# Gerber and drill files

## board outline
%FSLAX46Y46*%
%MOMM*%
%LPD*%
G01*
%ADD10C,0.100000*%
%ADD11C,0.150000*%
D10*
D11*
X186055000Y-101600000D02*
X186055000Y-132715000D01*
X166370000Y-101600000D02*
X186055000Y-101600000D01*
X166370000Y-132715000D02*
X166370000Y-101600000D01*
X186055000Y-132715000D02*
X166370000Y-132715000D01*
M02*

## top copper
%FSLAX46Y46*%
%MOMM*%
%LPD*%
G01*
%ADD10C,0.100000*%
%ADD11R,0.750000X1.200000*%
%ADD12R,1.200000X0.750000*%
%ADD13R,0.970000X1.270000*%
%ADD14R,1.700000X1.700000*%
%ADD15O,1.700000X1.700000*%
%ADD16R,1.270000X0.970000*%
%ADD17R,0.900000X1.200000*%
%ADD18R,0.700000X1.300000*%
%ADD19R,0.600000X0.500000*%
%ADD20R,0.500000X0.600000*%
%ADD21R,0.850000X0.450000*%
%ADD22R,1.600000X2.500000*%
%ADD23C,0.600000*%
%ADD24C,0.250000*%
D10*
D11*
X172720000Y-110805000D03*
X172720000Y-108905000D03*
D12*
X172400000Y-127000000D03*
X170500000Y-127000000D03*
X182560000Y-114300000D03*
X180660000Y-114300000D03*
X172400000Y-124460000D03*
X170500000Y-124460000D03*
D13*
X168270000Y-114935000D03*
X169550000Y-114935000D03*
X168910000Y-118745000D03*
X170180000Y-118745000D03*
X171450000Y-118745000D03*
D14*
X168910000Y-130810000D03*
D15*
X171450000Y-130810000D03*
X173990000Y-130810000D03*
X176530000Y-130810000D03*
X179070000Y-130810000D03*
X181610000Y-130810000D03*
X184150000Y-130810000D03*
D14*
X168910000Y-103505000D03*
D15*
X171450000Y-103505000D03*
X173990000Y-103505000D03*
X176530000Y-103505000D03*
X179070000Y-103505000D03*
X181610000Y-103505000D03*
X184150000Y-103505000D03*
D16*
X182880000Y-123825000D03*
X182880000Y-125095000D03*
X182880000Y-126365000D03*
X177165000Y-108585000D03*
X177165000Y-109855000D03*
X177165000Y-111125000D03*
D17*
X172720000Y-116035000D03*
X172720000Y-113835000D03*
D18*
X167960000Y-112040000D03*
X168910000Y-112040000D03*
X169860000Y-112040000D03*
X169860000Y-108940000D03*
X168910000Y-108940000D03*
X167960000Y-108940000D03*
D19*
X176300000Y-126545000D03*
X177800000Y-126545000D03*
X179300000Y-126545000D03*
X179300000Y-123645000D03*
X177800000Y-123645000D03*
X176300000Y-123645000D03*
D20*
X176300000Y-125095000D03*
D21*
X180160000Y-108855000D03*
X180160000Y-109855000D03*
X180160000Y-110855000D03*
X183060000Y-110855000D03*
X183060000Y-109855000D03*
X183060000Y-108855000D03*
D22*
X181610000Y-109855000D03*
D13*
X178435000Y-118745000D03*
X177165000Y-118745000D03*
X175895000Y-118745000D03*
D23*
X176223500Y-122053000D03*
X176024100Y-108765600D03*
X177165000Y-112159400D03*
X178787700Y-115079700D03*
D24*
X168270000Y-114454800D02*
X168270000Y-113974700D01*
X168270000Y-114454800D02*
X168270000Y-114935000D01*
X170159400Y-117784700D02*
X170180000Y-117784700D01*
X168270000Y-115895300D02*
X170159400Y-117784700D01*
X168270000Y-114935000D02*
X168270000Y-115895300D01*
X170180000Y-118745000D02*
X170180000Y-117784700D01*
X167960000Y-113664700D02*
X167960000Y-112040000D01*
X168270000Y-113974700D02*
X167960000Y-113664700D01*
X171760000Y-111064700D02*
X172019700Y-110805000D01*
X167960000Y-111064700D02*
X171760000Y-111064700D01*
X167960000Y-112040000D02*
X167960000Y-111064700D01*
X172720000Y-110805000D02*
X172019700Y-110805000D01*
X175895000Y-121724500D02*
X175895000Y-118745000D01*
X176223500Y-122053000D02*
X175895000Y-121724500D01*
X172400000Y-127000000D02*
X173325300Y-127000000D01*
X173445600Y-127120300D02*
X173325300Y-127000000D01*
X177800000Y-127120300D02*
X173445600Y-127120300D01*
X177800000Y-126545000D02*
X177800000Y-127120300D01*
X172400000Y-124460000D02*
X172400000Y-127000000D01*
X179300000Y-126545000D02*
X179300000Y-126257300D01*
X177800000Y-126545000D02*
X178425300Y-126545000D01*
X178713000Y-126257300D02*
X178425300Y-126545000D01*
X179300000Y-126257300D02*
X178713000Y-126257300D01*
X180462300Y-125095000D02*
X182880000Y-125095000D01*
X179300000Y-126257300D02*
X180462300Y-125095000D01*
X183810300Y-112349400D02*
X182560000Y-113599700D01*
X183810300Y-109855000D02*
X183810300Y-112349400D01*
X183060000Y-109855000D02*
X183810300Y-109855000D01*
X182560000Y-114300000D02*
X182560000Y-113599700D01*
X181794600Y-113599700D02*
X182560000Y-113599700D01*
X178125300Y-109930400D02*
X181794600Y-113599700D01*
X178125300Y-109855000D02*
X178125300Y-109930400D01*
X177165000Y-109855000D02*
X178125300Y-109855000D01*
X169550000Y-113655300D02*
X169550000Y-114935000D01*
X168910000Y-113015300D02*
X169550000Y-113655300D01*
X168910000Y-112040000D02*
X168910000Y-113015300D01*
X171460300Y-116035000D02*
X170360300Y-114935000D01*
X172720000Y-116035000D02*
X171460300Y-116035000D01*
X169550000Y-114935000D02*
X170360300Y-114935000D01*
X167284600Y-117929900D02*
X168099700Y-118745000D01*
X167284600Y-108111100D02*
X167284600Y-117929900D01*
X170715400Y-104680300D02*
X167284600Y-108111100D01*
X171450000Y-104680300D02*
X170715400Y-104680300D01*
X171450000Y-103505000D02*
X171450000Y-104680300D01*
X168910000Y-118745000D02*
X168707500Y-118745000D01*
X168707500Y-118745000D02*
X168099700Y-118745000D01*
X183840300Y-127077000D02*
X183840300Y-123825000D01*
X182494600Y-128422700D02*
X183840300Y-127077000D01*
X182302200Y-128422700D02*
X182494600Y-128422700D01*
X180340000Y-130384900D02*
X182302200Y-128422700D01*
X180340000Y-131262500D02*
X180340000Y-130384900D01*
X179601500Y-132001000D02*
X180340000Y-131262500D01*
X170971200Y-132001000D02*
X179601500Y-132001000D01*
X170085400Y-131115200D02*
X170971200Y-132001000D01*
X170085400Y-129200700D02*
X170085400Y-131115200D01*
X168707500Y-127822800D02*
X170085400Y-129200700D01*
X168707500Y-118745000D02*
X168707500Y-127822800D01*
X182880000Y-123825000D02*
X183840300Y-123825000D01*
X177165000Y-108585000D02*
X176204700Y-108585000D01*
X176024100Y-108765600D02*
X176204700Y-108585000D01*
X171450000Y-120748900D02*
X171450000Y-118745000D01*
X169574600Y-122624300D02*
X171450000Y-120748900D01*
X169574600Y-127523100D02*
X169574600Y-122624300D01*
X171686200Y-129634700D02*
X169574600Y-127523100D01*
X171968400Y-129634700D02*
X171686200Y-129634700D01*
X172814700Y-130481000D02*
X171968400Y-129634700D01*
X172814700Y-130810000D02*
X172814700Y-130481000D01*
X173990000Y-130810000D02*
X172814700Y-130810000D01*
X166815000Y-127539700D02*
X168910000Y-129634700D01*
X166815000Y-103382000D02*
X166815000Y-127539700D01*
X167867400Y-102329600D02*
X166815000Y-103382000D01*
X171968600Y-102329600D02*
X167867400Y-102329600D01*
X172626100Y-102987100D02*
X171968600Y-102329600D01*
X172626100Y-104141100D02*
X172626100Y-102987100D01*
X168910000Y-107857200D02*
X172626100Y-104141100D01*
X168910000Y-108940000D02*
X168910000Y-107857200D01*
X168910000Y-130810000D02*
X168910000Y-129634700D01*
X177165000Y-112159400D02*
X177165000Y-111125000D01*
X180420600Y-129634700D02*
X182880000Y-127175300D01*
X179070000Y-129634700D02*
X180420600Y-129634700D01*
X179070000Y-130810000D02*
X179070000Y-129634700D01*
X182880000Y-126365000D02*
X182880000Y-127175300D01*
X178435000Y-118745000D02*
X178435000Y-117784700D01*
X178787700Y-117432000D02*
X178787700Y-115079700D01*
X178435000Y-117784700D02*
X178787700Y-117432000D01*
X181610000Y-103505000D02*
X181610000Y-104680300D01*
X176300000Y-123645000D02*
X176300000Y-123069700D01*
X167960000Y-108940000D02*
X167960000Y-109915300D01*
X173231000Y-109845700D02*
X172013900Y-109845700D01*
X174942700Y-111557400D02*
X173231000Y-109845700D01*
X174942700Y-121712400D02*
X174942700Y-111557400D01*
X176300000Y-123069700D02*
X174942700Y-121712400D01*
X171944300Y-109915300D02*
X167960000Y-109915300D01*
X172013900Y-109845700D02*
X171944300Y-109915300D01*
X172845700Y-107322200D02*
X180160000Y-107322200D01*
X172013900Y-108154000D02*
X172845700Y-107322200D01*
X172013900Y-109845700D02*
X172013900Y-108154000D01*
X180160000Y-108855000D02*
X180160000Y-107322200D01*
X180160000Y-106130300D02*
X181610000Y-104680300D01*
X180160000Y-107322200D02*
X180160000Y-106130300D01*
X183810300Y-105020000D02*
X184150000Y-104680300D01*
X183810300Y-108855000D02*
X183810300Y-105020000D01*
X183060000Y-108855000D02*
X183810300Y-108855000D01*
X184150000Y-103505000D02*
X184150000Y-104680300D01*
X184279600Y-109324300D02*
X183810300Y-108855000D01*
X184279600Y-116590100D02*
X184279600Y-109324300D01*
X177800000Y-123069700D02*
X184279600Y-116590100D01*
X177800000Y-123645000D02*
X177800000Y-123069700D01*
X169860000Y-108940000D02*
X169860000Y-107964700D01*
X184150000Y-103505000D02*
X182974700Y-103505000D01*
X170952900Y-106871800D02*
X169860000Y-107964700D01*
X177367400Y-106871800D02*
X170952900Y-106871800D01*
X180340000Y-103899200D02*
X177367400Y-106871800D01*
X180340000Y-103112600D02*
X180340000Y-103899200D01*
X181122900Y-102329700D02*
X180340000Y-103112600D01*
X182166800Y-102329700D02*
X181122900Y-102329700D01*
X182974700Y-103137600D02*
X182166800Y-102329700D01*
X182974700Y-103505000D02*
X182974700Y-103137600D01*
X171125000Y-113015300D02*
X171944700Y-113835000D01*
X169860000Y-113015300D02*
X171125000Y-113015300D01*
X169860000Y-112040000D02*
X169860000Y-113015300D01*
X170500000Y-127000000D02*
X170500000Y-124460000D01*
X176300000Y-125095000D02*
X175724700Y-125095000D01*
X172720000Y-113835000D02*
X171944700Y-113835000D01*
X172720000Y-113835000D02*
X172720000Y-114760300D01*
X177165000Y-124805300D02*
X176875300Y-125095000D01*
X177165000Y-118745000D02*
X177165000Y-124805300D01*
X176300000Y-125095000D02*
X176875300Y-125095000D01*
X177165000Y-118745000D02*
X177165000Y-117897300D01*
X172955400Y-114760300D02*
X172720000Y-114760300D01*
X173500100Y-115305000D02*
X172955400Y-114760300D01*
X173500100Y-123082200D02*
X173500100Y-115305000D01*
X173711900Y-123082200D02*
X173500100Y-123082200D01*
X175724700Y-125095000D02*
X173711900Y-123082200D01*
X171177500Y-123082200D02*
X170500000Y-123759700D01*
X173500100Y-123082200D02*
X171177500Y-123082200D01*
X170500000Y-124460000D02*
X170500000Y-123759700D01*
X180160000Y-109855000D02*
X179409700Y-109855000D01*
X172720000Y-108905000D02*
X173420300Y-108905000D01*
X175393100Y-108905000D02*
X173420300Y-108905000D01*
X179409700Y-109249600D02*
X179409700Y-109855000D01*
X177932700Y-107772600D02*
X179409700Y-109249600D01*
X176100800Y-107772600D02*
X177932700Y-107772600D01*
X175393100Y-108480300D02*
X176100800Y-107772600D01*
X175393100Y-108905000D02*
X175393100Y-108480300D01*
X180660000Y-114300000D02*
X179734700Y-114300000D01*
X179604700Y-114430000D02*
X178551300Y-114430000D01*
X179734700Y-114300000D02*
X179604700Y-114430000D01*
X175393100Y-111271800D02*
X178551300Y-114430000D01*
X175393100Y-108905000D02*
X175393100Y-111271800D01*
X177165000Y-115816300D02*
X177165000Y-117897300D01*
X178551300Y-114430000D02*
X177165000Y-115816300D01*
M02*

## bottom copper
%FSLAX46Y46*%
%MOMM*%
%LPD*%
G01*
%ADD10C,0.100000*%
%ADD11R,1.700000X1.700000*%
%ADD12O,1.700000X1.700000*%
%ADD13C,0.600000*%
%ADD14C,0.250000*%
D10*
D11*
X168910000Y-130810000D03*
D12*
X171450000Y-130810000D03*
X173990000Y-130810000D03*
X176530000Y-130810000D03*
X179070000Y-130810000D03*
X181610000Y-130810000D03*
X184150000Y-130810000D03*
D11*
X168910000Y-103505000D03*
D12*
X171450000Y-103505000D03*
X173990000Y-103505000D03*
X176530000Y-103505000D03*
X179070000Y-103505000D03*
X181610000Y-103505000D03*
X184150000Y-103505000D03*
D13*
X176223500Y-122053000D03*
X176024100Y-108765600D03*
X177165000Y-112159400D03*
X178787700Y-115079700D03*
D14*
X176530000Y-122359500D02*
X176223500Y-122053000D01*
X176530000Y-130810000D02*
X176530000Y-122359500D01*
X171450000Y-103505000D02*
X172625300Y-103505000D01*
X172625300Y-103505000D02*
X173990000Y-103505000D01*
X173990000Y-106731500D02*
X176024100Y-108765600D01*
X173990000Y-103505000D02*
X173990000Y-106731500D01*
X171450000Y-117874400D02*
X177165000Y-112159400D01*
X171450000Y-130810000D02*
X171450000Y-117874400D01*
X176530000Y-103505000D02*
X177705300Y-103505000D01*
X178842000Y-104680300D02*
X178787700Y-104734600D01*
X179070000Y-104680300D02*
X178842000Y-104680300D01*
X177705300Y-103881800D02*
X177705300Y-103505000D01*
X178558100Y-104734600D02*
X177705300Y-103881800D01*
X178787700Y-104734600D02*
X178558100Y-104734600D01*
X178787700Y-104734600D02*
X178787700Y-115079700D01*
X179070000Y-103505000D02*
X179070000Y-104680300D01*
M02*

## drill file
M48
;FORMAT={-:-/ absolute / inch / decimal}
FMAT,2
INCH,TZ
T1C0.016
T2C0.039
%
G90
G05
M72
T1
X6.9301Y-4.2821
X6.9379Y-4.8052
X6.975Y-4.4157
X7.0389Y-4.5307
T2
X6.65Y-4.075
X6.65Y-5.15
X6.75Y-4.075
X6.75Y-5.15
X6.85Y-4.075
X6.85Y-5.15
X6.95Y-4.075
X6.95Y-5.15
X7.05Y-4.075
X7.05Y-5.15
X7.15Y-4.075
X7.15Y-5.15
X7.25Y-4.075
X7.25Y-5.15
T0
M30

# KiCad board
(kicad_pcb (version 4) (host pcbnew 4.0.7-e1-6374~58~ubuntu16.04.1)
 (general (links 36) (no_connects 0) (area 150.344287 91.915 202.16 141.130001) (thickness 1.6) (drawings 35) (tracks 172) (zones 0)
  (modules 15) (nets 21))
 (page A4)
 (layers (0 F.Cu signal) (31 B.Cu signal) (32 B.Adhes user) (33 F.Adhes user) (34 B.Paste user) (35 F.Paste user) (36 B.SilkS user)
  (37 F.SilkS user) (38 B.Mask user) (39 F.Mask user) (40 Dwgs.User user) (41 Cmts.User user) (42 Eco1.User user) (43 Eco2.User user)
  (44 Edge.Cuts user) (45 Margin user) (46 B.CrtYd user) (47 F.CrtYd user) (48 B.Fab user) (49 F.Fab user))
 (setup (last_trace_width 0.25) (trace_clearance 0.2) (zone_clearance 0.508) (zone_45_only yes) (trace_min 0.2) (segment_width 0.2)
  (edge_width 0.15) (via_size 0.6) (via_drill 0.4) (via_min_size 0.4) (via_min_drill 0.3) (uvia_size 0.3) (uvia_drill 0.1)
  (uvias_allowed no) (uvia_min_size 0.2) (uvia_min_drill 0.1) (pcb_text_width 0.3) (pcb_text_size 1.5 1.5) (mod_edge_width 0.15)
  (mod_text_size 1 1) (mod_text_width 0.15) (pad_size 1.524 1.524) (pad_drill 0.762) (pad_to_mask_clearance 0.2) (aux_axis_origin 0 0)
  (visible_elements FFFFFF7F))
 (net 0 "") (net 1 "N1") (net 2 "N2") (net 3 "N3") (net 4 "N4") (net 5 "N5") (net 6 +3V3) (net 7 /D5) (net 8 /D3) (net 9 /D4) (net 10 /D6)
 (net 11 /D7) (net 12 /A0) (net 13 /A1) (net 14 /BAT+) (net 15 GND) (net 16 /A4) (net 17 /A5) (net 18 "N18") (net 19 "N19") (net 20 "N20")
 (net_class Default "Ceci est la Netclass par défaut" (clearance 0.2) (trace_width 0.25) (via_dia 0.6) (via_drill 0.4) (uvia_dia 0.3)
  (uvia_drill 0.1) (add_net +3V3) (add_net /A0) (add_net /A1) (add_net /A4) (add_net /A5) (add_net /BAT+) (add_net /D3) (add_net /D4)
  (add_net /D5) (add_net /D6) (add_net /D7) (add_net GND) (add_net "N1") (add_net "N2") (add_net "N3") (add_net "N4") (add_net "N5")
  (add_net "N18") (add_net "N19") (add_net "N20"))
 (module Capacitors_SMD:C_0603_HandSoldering (layer F.Cu) (at 172.72 109.855 90)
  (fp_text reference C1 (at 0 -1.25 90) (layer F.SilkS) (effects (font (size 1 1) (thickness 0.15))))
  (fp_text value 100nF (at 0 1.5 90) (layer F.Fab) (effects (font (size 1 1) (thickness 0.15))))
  (pad 1 smd rect (at -0.95 0 90) (size 1.2 0.75) (layers F.Cu F.Paste F.Mask) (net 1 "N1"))
  (pad 2 smd rect (at 0.95 0 90) (size 1.2 0.75) (layers F.Cu F.Paste F.Mask) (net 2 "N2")))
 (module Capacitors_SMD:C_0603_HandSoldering (layer F.Cu) (at 171.45 127 180)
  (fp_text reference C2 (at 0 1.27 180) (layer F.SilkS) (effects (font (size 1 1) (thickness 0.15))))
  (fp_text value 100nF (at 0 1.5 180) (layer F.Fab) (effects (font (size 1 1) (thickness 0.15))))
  (pad 1 smd rect (at -0.95 0 180) (size 1.2 0.75) (layers F.Cu F.Paste F.Mask) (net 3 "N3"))
  (pad 2 smd rect (at 0.95 0 180) (size 1.2 0.75) (layers F.Cu F.Paste F.Mask) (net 2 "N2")))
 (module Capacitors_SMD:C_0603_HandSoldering (layer F.Cu) (at 181.61 114.3 180)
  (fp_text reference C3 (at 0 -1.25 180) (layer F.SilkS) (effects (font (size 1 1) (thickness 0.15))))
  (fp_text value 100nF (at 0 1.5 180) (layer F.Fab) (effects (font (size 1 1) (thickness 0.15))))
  (pad 1 smd rect (at -0.95 0 180) (size 1.2 0.75) (layers F.Cu F.Paste F.Mask) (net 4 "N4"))
  (pad 2 smd rect (at 0.95 0 180) (size 1.2 0.75) (layers F.Cu F.Paste F.Mask) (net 2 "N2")))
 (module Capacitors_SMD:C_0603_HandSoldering (layer F.Cu) (at 171.45 124.46 180)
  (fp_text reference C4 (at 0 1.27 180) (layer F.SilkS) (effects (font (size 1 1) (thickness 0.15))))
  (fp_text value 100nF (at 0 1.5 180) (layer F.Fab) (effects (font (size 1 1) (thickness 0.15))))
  (pad 1 smd rect (at -0.95 0 180) (size 1.2 0.75) (layers F.Cu F.Paste F.Mask) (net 3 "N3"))
  (pad 2 smd rect (at 0.95 0 180) (size 1.2 0.75) (layers F.Cu F.Paste F.Mask) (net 2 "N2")))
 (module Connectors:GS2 (layer F.Cu) (at 168.91 114.935 90)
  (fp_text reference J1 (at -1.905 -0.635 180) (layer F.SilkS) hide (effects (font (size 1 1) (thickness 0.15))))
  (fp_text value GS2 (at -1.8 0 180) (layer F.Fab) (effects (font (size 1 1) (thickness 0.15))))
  (pad 1 smd rect (at 0 -0.64 90) (size 1.27 0.97) (layers F.Cu F.Paste F.Mask) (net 1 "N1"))
  (pad 2 smd rect (at 0 0.64 90) (size 1.27 0.97) (layers F.Cu F.Paste F.Mask) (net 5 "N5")))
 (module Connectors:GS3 (layer F.Cu) (at 170.18 118.745 90)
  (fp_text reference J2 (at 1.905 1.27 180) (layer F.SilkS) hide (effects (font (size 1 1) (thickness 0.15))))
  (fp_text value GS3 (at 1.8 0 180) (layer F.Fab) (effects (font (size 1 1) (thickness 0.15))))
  (pad 1 smd rect (at 0 -1.27 90) (size 1.27 0.97) (layers F.Cu F.Paste F.Mask) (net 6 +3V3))
  (pad 2 smd rect (at 0 0 90) (size 1.27 0.97) (layers F.Cu F.Paste F.Mask) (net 1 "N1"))
  (pad 3 smd rect (at 0 1.27 90) (size 1.27 0.97) (layers F.Cu F.Paste F.Mask) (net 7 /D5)))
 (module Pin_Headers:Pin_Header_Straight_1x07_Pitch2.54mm (layer B.Cu) (at 168.91 130.81 270)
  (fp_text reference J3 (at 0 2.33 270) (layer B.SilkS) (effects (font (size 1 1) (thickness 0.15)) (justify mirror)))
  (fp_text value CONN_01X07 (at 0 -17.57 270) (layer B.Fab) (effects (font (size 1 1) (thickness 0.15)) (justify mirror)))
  (pad 1 thru_hole rect (at 0 0 270) (size 1.7 1.7) (drill 1) (layers *.Cu *.Mask) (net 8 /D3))
  (pad 2 thru_hole oval (at 0 -2.54 270) (size 1.7 1.7) (drill 1) (layers *.Cu *.Mask) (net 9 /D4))
  (pad 3 thru_hole oval (at 0 -5.08 270) (size 1.7 1.7) (drill 1) (layers *.Cu *.Mask) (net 7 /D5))
  (pad 4 thru_hole oval (at 0 -7.62 270) (size 1.7 1.7) (drill 1) (layers *.Cu *.Mask) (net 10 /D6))
  (pad 5 thru_hole oval (at 0 -10.16 270) (size 1.7 1.7) (drill 1) (layers *.Cu *.Mask) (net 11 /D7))
  (pad 6 thru_hole oval (at 0 -12.7 270) (size 1.7 1.7) (drill 1) (layers *.Cu *.Mask) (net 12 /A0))
  (pad 7 thru_hole oval (at 0 -15.24 270) (size 1.7 1.7) (drill 1) (layers *.Cu *.Mask) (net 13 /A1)))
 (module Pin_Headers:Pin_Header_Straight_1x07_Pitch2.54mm (layer B.Cu) (at 168.91 103.505 270)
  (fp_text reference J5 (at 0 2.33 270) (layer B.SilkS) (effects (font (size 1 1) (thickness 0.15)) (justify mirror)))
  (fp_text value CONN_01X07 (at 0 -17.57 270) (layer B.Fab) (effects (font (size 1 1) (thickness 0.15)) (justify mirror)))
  (pad 1 thru_hole rect (at 0 0 270) (size 1.7 1.7) (drill 1) (layers *.Cu *.Mask) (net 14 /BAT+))
  (pad 2 thru_hole oval (at 0 -2.54 270) (size 1.7 1.7) (drill 1) (layers *.Cu *.Mask) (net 6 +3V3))
  (pad 3 thru_hole oval (at 0 -5.08 270) (size 1.7 1.7) (drill 1) (layers *.Cu *.Mask) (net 6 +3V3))
  (pad 4 thru_hole oval (at 0 -7.62 270) (size 1.7 1.7) (drill 1) (layers *.Cu *.Mask) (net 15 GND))
  (pad 5 thru_hole oval (at 0 -10.16 270) (size 1.7 1.7) (drill 1) (layers *.Cu *.Mask) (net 15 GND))
  (pad 6 thru_hole oval (at 0 -12.7 270) (size 1.7 1.7) (drill 1) (layers *.Cu *.Mask) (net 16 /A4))
  (pad 7 thru_hole oval (at 0 -15.24 270) (size 1.7 1.7) (drill 1) (layers *.Cu *.Mask) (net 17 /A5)))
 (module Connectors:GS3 (layer F.Cu) (at 182.88 125.095)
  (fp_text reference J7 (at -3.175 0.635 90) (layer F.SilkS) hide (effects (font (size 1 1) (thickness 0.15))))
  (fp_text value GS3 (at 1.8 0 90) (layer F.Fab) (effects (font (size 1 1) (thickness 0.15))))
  (pad 1 smd rect (at 0 -1.27) (size 1.27 0.97) (layers F.Cu F.Paste F.Mask) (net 6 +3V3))
  (pad 2 smd rect (at 0 0) (size 1.27 0.97) (layers F.Cu F.Paste F.Mask) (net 3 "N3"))
  (pad 3 smd rect (at 0 1.27) (size 1.27 0.97) (layers F.Cu F.Paste F.Mask) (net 11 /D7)))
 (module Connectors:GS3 (layer F.Cu) (at 177.165 109.855)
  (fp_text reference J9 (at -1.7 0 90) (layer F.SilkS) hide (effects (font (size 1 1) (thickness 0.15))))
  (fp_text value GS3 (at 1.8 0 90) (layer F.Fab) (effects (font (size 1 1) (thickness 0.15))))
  (pad 1 smd rect (at 0 -1.27) (size 1.27 0.97) (layers F.Cu F.Paste F.Mask) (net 6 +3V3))
  (pad 2 smd rect (at 0 0) (size 1.27 0.97) (layers F.Cu F.Paste F.Mask) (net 4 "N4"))
  (pad 3 smd rect (at 0 1.27) (size 1.27 0.97) (layers F.Cu F.Paste F.Mask) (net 9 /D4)))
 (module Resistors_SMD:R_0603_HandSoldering (layer F.Cu) (at 172.72 114.935 90)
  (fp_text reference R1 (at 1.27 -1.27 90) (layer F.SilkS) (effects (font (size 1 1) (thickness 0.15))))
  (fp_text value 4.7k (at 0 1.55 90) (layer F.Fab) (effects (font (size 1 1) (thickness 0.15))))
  (pad 1 smd rect (at -1.1 0 90) (size 1.2 0.9) (layers F.Cu F.Paste F.Mask) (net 5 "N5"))
  (pad 2 smd rect (at 1.1 0 90) (size 1.2 0.9) (layers F.Cu F.Paste F.Mask) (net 2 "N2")))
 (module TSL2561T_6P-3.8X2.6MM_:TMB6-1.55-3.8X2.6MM (layer F.Cu) (at 168.91 110.49 90)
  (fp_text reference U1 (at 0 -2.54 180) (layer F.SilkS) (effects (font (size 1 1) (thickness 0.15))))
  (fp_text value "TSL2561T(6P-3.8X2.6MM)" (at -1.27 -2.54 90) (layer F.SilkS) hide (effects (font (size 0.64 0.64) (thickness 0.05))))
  (pad 1 smd rect (at -1.55 -0.95 90) (size 1.3 0.7) (layers F.Cu F.Paste F.Mask) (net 1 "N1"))
  (pad 2 smd rect (at -1.55 0 90) (size 1.3 0.7) (layers F.Cu F.Paste F.Mask) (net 5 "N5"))
  (pad 3 smd rect (at -1.55 0.95 90) (size 1.3 0.7) (layers F.Cu F.Paste F.Mask) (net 2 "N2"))
  (pad 4 smd rect (at 1.55 0.95 270) (size 1.3 0.7) (layers F.Cu F.Paste F.Mask) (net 17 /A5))
  (pad 5 smd rect (at 1.55 0 270) (size 1.3 0.7) (layers F.Cu F.Paste F.Mask) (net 8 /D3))
  (pad 6 smd rect (at 1.55 -0.95 270) (size 1.3 0.7) (layers F.Cu F.Paste F.Mask) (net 16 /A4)))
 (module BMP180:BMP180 (layer F.Cu) (at 177.8 125.095 180)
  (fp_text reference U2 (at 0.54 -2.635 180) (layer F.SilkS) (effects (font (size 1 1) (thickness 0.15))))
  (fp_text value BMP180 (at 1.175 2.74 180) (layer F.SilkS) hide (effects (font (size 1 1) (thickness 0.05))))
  (pad 1 smd rect (at 1.5 -1.45 270) (size 0.5 0.6) (layers F.Cu F.Paste F.Mask))
  (pad 2 smd rect (at 0 -1.45 270) (size 0.5 0.6) (layers F.Cu F.Paste F.Mask) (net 3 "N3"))
  (pad 3 smd rect (at -1.5 -1.45 270) (size 0.5 0.6) (layers F.Cu F.Paste F.Mask) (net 3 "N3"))
  (pad 4 smd rect (at -1.5 1.45 270) (size 0.5 0.6) (layers F.Cu F.Paste F.Mask))
  (pad 5 smd rect (at 0 1.45 270) (size 0.5 0.6) (layers F.Cu F.Paste F.Mask) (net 17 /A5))
  (pad 6 smd rect (at 1.5 1.45 270) (size 0.5 0.6) (layers F.Cu F.Paste F.Mask) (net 16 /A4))
  (pad 7 smd rect (at 1.5 0) (size 0.5 0.6) (layers F.Cu F.Paste F.Mask) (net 2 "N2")))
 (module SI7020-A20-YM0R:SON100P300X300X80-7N (layer F.Cu) (at 181.61 109.855)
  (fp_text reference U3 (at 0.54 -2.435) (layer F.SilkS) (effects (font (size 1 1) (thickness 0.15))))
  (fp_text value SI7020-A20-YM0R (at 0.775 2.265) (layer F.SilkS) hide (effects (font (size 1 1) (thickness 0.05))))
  (pad 1 smd rect (at -1.45 -1) (size 0.85 0.45) (layers F.Cu F.Paste F.Mask) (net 16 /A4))
  (pad 2 smd rect (at -1.45 0) (size 0.85 0.45) (layers F.Cu F.Paste F.Mask) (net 2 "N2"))
  (pad 3 smd rect (at -1.45 1) (size 0.85 0.45) (layers F.Cu F.Paste F.Mask) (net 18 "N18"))
  (pad 4 smd rect (at 1.45 1 180) (size 0.85 0.45) (layers F.Cu F.Paste F.Mask) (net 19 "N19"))
  (pad 5 smd rect (at 1.45 0 180) (size 0.85 0.45) (layers F.Cu F.Paste F.Mask) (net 4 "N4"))
  (pad 6 smd rect (at 1.45 -1 180) (size 0.85 0.45) (layers F.Cu F.Paste F.Mask) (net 17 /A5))
  (pad 7 smd rect (at 0 0) (size 1.6 2.5) (layers F.Cu F.Paste F.Mask) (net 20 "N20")))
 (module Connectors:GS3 (layer F.Cu) (at 177.165 118.745 270)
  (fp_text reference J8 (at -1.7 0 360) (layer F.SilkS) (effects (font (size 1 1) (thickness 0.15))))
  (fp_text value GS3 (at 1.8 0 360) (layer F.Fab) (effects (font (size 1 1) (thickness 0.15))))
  (pad 1 smd rect (at 0 -1.27 270) (size 1.27 0.97) (layers F.Cu F.Paste F.Mask) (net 15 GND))
  (pad 2 smd rect (at 0 0 270) (size 1.27 0.97) (layers F.Cu F.Paste F.Mask) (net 2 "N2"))
  (pad 3 smd rect (at 0 1.27 270) (size 1.27 0.97) (layers F.Cu F.Paste F.Mask) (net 10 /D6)))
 (gr_line (start 186.055 101.6) (end 186.055 132.715) (angle 90) (layer Edge.Cuts) (width 0.15))
 (gr_line (start 166.37 101.6) (end 186.055 101.6) (angle 90) (layer Edge.Cuts) (width 0.15))
 (gr_line (start 166.37 132.715) (end 166.37 101.6) (angle 90) (layer Edge.Cuts) (width 0.15))
 (gr_line (start 186.055 132.715) (end 166.37 132.715) (angle 90) (layer Edge.Cuts) (width 0.15))
 (segment (start 168.27 114.4548) (end 168.27 113.9747) (width 0.25) (layer F.Cu) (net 1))
 (segment (start 168.27 114.4548) (end 168.27 114.935) (width 0.25) (layer F.Cu) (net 1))
 (segment (start 170.1594 117.7847) (end 170.18 117.7847) (width 0.25) (layer F.Cu) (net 1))
 (segment (start 168.27 115.8953) (end 170.1594 117.7847) (width 0.25) (layer F.Cu) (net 1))
 (segment (start 168.27 114.935) (end 168.27 115.8953) (width 0.25) (layer F.Cu) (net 1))
 (segment (start 170.18 118.745) (end 170.18 117.7847) (width 0.25) (layer F.Cu) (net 1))
 (segment (start 167.96 113.6647) (end 167.96 112.04) (width 0.25) (layer F.Cu) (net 1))
 (segment (start 168.27 113.9747) (end 167.96 113.6647) (width 0.25) (layer F.Cu) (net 1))
 (segment (start 171.76 111.0647) (end 172.0197 110.805) (width 0.25) (layer F.Cu) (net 1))
 (segment (start 167.96 111.0647) (end 171.76 111.0647) (width 0.25) (layer F.Cu) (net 1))
 (segment (start 167.96 112.04) (end 167.96 111.0647) (width 0.25) (layer F.Cu) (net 1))
 (segment (start 172.72 110.805) (end 172.0197 110.805) (width 0.25) (layer F.Cu) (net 1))
 (via (at 176.2235 122.053) (size 0.6) (layers F.Cu B.Cu) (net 10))
 (segment (start 176.53 122.3595) (end 176.2235 122.053) (width 0.25) (layer B.Cu) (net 10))
 (segment (start 176.53 130.81) (end 176.53 122.3595) (width 0.25) (layer B.Cu) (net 10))
 (segment (start 175.895 121.7245) (end 175.895 118.745) (width 0.25) (layer F.Cu) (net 10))
 (segment (start 176.2235 122.053) (end 175.895 121.7245) (width 0.25) (layer F.Cu) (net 10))
 (segment (start 172.4 127) (end 173.3253 127) (width 0.25) (layer F.Cu) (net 3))
 (segment (start 173.4456 127.1203) (end 173.3253 127) (width 0.25) (layer F.Cu) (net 3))
 (segment (start 177.8 127.1203) (end 173.4456 127.1203) (width 0.25) (layer F.Cu) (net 3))
 (segment (start 177.8 126.545) (end 177.8 127.1203) (width 0.25) (layer F.Cu) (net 3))
 (segment (start 172.4 124.46) (end 172.4 127) (width 0.25) (layer F.Cu) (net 3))
 (segment (start 179.3 126.545) (end 179.3 126.2573) (width 0.25) (layer F.Cu) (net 3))
 (segment (start 177.8 126.545) (end 178.4253 126.545) (width 0.25) (layer F.Cu) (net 3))
 (segment (start 178.713 126.2573) (end 178.4253 126.545) (width 0.25) (layer F.Cu) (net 3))
 (segment (start 179.3 126.2573) (end 178.713 126.2573) (width 0.25) (layer F.Cu) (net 3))
 (segment (start 180.4623 125.095) (end 182.88 125.095) (width 0.25) (layer F.Cu) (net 3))
 (segment (start 179.3 126.2573) (end 180.4623 125.095) (width 0.25) (layer F.Cu) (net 3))
 (segment (start 183.8103 112.3494) (end 182.56 113.5997) (width 0.25) (layer F.Cu) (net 4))
 (segment (start 183.8103 109.855) (end 183.8103 112.3494) (width 0.25) (layer F.Cu) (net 4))
 (segment (start 183.06 109.855) (end 183.8103 109.855) (width 0.25) (layer F.Cu) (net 4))
 (segment (start 182.56 114.3) (end 182.56 113.5997) (width 0.25) (layer F.Cu) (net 4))
 (segment (start 181.7946 113.5997) (end 182.56 113.5997) (width 0.25) (layer F.Cu) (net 4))
 (segment (start 178.1253 109.9304) (end 181.7946 113.5997) (width 0.25) (layer F.Cu) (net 4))
 (segment (start 178.1253 109.855) (end 178.1253 109.9304) (width 0.25) (layer F.Cu) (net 4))
 (segment (start 177.165 109.855) (end 178.1253 109.855) (width 0.25) (layer F.Cu) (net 4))
 (segment (start 169.55 113.6553) (end 169.55 114.935) (width 0.25) (layer F.Cu) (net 5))
 (segment (start 168.91 113.0153) (end 169.55 113.6553) (width 0.25) (layer F.Cu) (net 5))
 (segment (start 168.91 112.04) (end 168.91 113.0153) (width 0.25) (layer F.Cu) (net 5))
 (segment (start 171.4603 116.035) (end 170.3603 114.935) (width 0.25) (layer F.Cu) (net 5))
 (segment (start 172.72 116.035) (end 171.4603 116.035) (width 0.25) (layer F.Cu) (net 5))
 (segment (start 169.55 114.935) (end 170.3603 114.935) (width 0.25) (layer F.Cu) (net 5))
 (via (at 176.0241 108.7656) (size 0.6) (layers F.Cu B.Cu) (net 6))
 (segment (start 171.45 103.505) (end 172.6253 103.505) (width 0.25) (layer B.Cu) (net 6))
 (segment (start 167.2846 117.9299) (end 168.0997 118.745) (width 0.25) (layer F.Cu) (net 6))
 (segment (start 167.2846 108.1111) (end 167.2846 117.9299) (width 0.25) (layer F.Cu) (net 6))
 (segment (start 170.7154 104.6803) (end 167.2846 108.1111) (width 0.25) (layer F.Cu) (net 6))
 (segment (start 171.45 104.6803) (end 170.7154 104.6803) (width 0.25) (layer F.Cu) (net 6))
 (segment (start 171.45 103.505) (end 171.45 104.6803) (width 0.25) (layer F.Cu) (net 6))
 (segment (start 168.91 118.745) (end 168.7075 118.745) (width 0.25) (layer F.Cu) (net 6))
 (segment (start 168.7075 118.745) (end 168.0997 118.745) (width 0.25) (layer F.Cu) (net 6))
 (segment (start 183.8403 127.077) (end 183.8403 123.825) (width 0.25) (layer F.Cu) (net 6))
 (segment (start 182.4946 128.4227) (end 183.8403 127.077) (width 0.25) (layer F.Cu) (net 6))
 (segment (start 182.3022 128.4227) (end 182.4946 128.4227) (width 0.25) (layer F.Cu) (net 6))
 (segment (start 180.34 130.3849) (end 182.3022 128.4227) (width 0.25) (layer F.Cu) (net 6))
 (segment (start 180.34 131.2625) (end 180.34 130.3849) (width 0.25) (layer F.Cu) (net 6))
 (segment (start 179.6015 132.001) (end 180.34 131.2625) (width 0.25) (layer F.Cu) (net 6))
 (segment (start 170.9712 132.001) (end 179.6015 132.001) (width 0.25) (layer F.Cu) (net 6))
 (segment (start 170.0854 131.1152) (end 170.9712 132.001) (width 0.25) (layer F.Cu) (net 6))
 (segment (start 170.0854 129.2007) (end 170.0854 131.1152) (width 0.25) (layer F.Cu) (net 6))
 (segment (start 168.7075 127.8228) (end 170.0854 129.2007) (width 0.25) (layer F.Cu) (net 6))
 (segment (start 168.7075 118.745) (end 168.7075 127.8228) (width 0.25) (layer F.Cu) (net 6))
 (segment (start 182.88 123.825) (end 183.8403 123.825) (width 0.25) (layer F.Cu) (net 6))
 (segment (start 177.165 108.585) (end 176.2047 108.585) (width 0.25) (layer F.Cu) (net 6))
 (segment (start 176.0241 108.7656) (end 176.2047 108.585) (width 0.25) (layer F.Cu) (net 6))
 (segment (start 172.6253 103.505) (end 173.99 103.505) (width 0.25) (layer B.Cu) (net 6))
 (segment (start 173.99 106.7315) (end 176.0241 108.7656) (width 0.25) (layer B.Cu) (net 6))
 (segment (start 173.99 103.505) (end 173.99 106.7315) (width 0.25) (layer B.Cu) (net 6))
 (segment (start 171.45 120.7489) (end 171.45 118.745) (width 0.25) (layer F.Cu) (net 7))
 (segment (start 169.5746 122.6243) (end 171.45 120.7489) (width 0.25) (layer F.Cu) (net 7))
 (segment (start 169.5746 127.5231) (end 169.5746 122.6243) (width 0.25) (layer F.Cu) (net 7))
 (segment (start 171.6862 129.6347) (end 169.5746 127.5231) (width 0.25) (layer F.Cu) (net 7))
 (segment (start 171.9684 129.6347) (end 171.6862 129.6347) (width 0.25) (layer F.Cu) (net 7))
 (segment (start 172.8147 130.481) (end 171.9684 129.6347) (width 0.25) (layer F.Cu) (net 7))
 (segment (start 172.8147 130.81) (end 172.8147 130.481) (width 0.25) (layer F.Cu) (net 7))
 (segment (start 173.99 130.81) (end 172.8147 130.81) (width 0.25) (layer F.Cu) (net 7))
 (segment (start 166.815 127.5397) (end 168.91 129.6347) (width 0.25) (layer F.Cu) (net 8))
 (segment (start 166.815 103.382) (end 166.815 127.5397) (width 0.25) (layer F.Cu) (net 8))
 (segment (start 167.8674 102.3296) (end 166.815 103.382) (width 0.25) (layer F.Cu) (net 8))
 (segment (start 171.9686 102.3296) (end 167.8674 102.3296) (width 0.25) (layer F.Cu) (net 8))
 (segment (start 172.6261 102.9871) (end 171.9686 102.3296) (width 0.25) (layer F.Cu) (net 8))
 (segment (start 172.6261 104.1411) (end 172.6261 102.9871) (width 0.25) (layer F.Cu) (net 8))
 (segment (start 168.91 107.8572) (end 172.6261 104.1411) (width 0.25) (layer F.Cu) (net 8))
 (segment (start 168.91 108.94) (end 168.91 107.8572) (width 0.25) (layer F.Cu) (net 8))
 (segment (start 168.91 130.81) (end 168.91 129.6347) (width 0.25) (layer F.Cu) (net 8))
 (via (at 177.165 112.1594) (size 0.6) (layers F.Cu B.Cu) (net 9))
 (segment (start 171.45 117.8744) (end 177.165 112.1594) (width 0.25) (layer B.Cu) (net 9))
 (segment (start 171.45 130.81) (end 171.45 117.8744) (width 0.25) (layer B.Cu) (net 9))
 (segment (start 177.165 112.1594) (end 177.165 111.125) (width 0.25) (layer F.Cu) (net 9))
 (segment (start 180.4206 129.6347) (end 182.88 127.1753) (width 0.25) (layer F.Cu) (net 11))
 (segment (start 179.07 129.6347) (end 180.4206 129.6347) (width 0.25) (layer F.Cu) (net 11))
 (segment (start 179.07 130.81) (end 179.07 129.6347) (width 0.25) (layer F.Cu) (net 11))
 (segment (start 182.88 126.365) (end 182.88 127.1753) (width 0.25) (layer F.Cu) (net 11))
 (via (at 178.7877 115.0797) (size 0.6) (layers F.Cu B.Cu) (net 15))
 (segment (start 178.435 118.745) (end 178.435 117.7847) (width 0.25) (layer F.Cu) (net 15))
 (segment (start 176.53 103.505) (end 177.7053 103.505) (width 0.25) (layer B.Cu) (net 15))
 (segment (start 178.842 104.6803) (end 178.7877 104.7346) (width 0.25) (layer B.Cu) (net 15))
 (segment (start 179.07 104.6803) (end 178.842 104.6803) (width 0.25) (layer B.Cu) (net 15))
 (segment (start 177.7053 103.8818) (end 177.7053 103.505) (width 0.25) (layer B.Cu) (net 15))
 (segment (start 178.5581 104.7346) (end 177.7053 103.8818) (width 0.25) (layer B.Cu) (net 15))
 (segment (start 178.7877 104.7346) (end 178.5581 104.7346) (width 0.25) (layer B.Cu) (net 15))
 (segment (start 178.7877 104.7346) (end 178.7877 115.0797) (width 0.25) (layer B.Cu) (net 15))
 (segment (start 178.7877 117.432) (end 178.7877 115.0797) (width 0.25) (layer F.Cu) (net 15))
 (segment (start 178.435 117.7847) (end 178.7877 117.432) (width 0.25) (layer F.Cu) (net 15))
 (segment (start 179.07 103.505) (end 179.07 104.6803) (width 0.25) (layer B.Cu) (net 15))
 (segment (start 181.61 103.505) (end 181.61 104.6803) (width 0.25) (layer F.Cu) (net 16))
 (segment (start 176.3 123.645) (end 176.3 123.0697) (width 0.25) (layer F.Cu) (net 16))
 (segment (start 167.96 108.94) (end 167.96 109.9153) (width 0.25) (layer F.Cu) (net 16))
 (segment (start 173.231 109.8457) (end 172.0139 109.8457) (width 0.25) (layer F.Cu) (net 16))
 (segment (start 174.9427 111.5574) (end 173.231 109.8457) (width 0.25) (layer F.Cu) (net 16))
 (segment (start 174.9427 121.7124) (end 174.9427 111.5574) (width 0.25) (layer F.Cu) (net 16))
 (segment (start 176.3 123.0697) (end 174.9427 121.7124) (width 0.25) (layer F.Cu) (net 16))
 (segment (start 171.9443 109.9153) (end 167.96 109.9153) (width 0.25) (layer F.Cu) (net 16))
 (segment (start 172.0139 109.8457) (end 171.9443 109.9153) (width 0.25) (layer F.Cu) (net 16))
 (segment (start 172.8457 107.3222) (end 180.16 107.3222) (width 0.25) (layer F.Cu) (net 16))
 (segment (start 172.0139 108.154) (end 172.8457 107.3222) (width 0.25) (layer F.Cu) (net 16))
 (segment (start 172.0139 109.8457) (end 172.0139 108.154) (width 0.25) (layer F.Cu) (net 16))
 (segment (start 180.16 108.855) (end 180.16 107.3222) (width 0.25) (layer F.Cu) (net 16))
 (segment (start 180.16 106.1303) (end 181.61 104.6803) (width 0.25) (layer F.Cu) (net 16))
 (segment (start 180.16 107.3222) (end 180.16 106.1303) (width 0.25) (layer F.Cu) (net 16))
 (segment (start 183.8103 105.02) (end 184.15 104.6803) (width 0.25) (layer F.Cu) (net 17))
 (segment (start 183.8103 108.855) (end 183.8103 105.02) (width 0.25) (layer F.Cu) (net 17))
 (segment (start 183.06 108.855) (end 183.8103 108.855) (width 0.25) (layer F.Cu) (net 17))
 (segment (start 184.15 103.505) (end 184.15 104.6803) (width 0.25) (layer F.Cu) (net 17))
 (segment (start 184.2796 109.3243) (end 183.8103 108.855) (width 0.25) (layer F.Cu) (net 17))
 (segment (start 184.2796 116.5901) (end 184.2796 109.3243) (width 0.25) (layer F.Cu) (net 17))
 (segment (start 177.8 123.0697) (end 184.2796 116.5901) (width 0.25) (layer F.Cu) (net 17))
 (segment (start 177.8 123.645) (end 177.8 123.0697) (width 0.25) (layer F.Cu) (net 17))
 (segment (start 169.86 108.94) (end 169.86 107.9647) (width 0.25) (layer F.Cu) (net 17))
 (segment (start 184.15 103.505) (end 182.9747 103.505) (width 0.25) (layer F.Cu) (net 17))
 (segment (start 170.9529 106.8718) (end 169.86 107.9647) (width 0.25) (layer F.Cu) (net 17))
 (segment (start 177.3674 106.8718) (end 170.9529 106.8718) (width 0.25) (layer F.Cu) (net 17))
 (segment (start 180.34 103.8992) (end 177.3674 106.8718) (width 0.25) (layer F.Cu) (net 17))
 (segment (start 180.34 103.1126) (end 180.34 103.8992) (width 0.25) (layer F.Cu) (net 17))
 (segment (start 181.1229 102.3297) (end 180.34 103.1126) (width 0.25) (layer F.Cu) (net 17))
 (segment (start 182.1668 102.3297) (end 181.1229 102.3297) (width 0.25) (layer F.Cu) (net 17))
 (segment (start 182.9747 103.1376) (end 182.1668 102.3297) (width 0.25) (layer F.Cu) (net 17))
 (segment (start 182.9747 103.505) (end 182.9747 103.1376) (width 0.25) (layer F.Cu) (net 17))
 (segment (start 171.125 113.0153) (end 171.9447 113.835) (width 0.25) (layer F.Cu) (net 2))
 (segment (start 169.86 113.0153) (end 171.125 113.0153) (width 0.25) (layer F.Cu) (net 2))
 (segment (start 169.86 112.04) (end 169.86 113.0153) (width 0.25) (layer F.Cu) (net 2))
 (segment (start 170.5 127) (end 170.5 124.46) (width 0.25) (layer F.Cu) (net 2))
 (segment (start 176.3 125.095) (end 175.7247 125.095) (width 0.25) (layer F.Cu) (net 2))
 (segment (start 172.72 113.835) (end 171.9447 113.835) (width 0.25) (layer F.Cu) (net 2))
 (segment (start 172.72 113.835) (end 172.72 114.7603) (width 0.25) (layer F.Cu) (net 2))
 (segment (start 177.165 124.8053) (end 176.8753 125.095) (width 0.25) (layer F.Cu) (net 2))
 (segment (start 177.165 118.745) (end 177.165 124.8053) (width 0.25) (layer F.Cu) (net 2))
 (segment (start 176.3 125.095) (end 176.8753 125.095) (width 0.25) (layer F.Cu) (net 2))
 (segment (start 177.165 118.745) (end 177.165 117.8973) (width 0.25) (layer F.Cu) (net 2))
 (segment (start 172.9554 114.7603) (end 172.72 114.7603) (width 0.25) (layer F.Cu) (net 2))
 (segment (start 173.5001 115.305) (end 172.9554 114.7603) (width 0.25) (layer F.Cu) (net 2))
 (segment (start 173.5001 123.0822) (end 173.5001 115.305) (width 0.25) (layer F.Cu) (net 2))
 (segment (start 173.7119 123.0822) (end 173.5001 123.0822) (width 0.25) (layer F.Cu) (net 2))
 (segment (start 175.7247 125.095) (end 173.7119 123.0822) (width 0.25) (layer F.Cu) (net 2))
 (segment (start 171.1775 123.0822) (end 170.5 123.7597) (width 0.25) (layer F.Cu) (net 2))
 (segment (start 173.5001 123.0822) (end 171.1775 123.0822) (width 0.25) (layer F.Cu) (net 2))
 (segment (start 170.5 124.46) (end 170.5 123.7597) (width 0.25) (layer F.Cu) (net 2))
 (segment (start 180.16 109.855) (end 179.4097 109.855) (width 0.25) (layer F.Cu) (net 2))
 (segment (start 172.72 108.905) (end 173.4203 108.905) (width 0.25) (layer F.Cu) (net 2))
 (segment (start 175.3931 108.905) (end 173.4203 108.905) (width 0.25) (layer F.Cu) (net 2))
 (segment (start 179.4097 109.2496) (end 179.4097 109.855) (width 0.25) (layer F.Cu) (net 2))
 (segment (start 177.9327 107.7726) (end 179.4097 109.2496) (width 0.25) (layer F.Cu) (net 2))
 (segment (start 176.1008 107.7726) (end 177.9327 107.7726) (width 0.25) (layer F.Cu) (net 2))
 (segment (start 175.3931 108.4803) (end 176.1008 107.7726) (width 0.25) (layer F.Cu) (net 2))
 (segment (start 175.3931 108.905) (end 175.3931 108.4803) (width 0.25) (layer F.Cu) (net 2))
 (segment (start 180.66 114.3) (end 179.7347 114.3) (width 0.25) (layer F.Cu) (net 2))
 (segment (start 179.6047 114.43) (end 178.5513 114.43) (width 0.25) (layer F.Cu) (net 2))
 (segment (start 179.7347 114.3) (end 179.6047 114.43) (width 0.25) (layer F.Cu) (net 2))
 (segment (start 175.3931 111.2718) (end 178.5513 114.43) (width 0.25) (layer F.Cu) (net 2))
 (segment (start 175.3931 108.905) (end 175.3931 111.2718) (width 0.25) (layer F.Cu) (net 2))
 (segment (start 177.165 115.8163) (end 177.165 117.8973) (width 0.25) (layer F.Cu) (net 2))
 (segment (start 178.5513 114.43) (end 177.165 115.8163) (width 0.25) (layer F.Cu) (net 2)))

